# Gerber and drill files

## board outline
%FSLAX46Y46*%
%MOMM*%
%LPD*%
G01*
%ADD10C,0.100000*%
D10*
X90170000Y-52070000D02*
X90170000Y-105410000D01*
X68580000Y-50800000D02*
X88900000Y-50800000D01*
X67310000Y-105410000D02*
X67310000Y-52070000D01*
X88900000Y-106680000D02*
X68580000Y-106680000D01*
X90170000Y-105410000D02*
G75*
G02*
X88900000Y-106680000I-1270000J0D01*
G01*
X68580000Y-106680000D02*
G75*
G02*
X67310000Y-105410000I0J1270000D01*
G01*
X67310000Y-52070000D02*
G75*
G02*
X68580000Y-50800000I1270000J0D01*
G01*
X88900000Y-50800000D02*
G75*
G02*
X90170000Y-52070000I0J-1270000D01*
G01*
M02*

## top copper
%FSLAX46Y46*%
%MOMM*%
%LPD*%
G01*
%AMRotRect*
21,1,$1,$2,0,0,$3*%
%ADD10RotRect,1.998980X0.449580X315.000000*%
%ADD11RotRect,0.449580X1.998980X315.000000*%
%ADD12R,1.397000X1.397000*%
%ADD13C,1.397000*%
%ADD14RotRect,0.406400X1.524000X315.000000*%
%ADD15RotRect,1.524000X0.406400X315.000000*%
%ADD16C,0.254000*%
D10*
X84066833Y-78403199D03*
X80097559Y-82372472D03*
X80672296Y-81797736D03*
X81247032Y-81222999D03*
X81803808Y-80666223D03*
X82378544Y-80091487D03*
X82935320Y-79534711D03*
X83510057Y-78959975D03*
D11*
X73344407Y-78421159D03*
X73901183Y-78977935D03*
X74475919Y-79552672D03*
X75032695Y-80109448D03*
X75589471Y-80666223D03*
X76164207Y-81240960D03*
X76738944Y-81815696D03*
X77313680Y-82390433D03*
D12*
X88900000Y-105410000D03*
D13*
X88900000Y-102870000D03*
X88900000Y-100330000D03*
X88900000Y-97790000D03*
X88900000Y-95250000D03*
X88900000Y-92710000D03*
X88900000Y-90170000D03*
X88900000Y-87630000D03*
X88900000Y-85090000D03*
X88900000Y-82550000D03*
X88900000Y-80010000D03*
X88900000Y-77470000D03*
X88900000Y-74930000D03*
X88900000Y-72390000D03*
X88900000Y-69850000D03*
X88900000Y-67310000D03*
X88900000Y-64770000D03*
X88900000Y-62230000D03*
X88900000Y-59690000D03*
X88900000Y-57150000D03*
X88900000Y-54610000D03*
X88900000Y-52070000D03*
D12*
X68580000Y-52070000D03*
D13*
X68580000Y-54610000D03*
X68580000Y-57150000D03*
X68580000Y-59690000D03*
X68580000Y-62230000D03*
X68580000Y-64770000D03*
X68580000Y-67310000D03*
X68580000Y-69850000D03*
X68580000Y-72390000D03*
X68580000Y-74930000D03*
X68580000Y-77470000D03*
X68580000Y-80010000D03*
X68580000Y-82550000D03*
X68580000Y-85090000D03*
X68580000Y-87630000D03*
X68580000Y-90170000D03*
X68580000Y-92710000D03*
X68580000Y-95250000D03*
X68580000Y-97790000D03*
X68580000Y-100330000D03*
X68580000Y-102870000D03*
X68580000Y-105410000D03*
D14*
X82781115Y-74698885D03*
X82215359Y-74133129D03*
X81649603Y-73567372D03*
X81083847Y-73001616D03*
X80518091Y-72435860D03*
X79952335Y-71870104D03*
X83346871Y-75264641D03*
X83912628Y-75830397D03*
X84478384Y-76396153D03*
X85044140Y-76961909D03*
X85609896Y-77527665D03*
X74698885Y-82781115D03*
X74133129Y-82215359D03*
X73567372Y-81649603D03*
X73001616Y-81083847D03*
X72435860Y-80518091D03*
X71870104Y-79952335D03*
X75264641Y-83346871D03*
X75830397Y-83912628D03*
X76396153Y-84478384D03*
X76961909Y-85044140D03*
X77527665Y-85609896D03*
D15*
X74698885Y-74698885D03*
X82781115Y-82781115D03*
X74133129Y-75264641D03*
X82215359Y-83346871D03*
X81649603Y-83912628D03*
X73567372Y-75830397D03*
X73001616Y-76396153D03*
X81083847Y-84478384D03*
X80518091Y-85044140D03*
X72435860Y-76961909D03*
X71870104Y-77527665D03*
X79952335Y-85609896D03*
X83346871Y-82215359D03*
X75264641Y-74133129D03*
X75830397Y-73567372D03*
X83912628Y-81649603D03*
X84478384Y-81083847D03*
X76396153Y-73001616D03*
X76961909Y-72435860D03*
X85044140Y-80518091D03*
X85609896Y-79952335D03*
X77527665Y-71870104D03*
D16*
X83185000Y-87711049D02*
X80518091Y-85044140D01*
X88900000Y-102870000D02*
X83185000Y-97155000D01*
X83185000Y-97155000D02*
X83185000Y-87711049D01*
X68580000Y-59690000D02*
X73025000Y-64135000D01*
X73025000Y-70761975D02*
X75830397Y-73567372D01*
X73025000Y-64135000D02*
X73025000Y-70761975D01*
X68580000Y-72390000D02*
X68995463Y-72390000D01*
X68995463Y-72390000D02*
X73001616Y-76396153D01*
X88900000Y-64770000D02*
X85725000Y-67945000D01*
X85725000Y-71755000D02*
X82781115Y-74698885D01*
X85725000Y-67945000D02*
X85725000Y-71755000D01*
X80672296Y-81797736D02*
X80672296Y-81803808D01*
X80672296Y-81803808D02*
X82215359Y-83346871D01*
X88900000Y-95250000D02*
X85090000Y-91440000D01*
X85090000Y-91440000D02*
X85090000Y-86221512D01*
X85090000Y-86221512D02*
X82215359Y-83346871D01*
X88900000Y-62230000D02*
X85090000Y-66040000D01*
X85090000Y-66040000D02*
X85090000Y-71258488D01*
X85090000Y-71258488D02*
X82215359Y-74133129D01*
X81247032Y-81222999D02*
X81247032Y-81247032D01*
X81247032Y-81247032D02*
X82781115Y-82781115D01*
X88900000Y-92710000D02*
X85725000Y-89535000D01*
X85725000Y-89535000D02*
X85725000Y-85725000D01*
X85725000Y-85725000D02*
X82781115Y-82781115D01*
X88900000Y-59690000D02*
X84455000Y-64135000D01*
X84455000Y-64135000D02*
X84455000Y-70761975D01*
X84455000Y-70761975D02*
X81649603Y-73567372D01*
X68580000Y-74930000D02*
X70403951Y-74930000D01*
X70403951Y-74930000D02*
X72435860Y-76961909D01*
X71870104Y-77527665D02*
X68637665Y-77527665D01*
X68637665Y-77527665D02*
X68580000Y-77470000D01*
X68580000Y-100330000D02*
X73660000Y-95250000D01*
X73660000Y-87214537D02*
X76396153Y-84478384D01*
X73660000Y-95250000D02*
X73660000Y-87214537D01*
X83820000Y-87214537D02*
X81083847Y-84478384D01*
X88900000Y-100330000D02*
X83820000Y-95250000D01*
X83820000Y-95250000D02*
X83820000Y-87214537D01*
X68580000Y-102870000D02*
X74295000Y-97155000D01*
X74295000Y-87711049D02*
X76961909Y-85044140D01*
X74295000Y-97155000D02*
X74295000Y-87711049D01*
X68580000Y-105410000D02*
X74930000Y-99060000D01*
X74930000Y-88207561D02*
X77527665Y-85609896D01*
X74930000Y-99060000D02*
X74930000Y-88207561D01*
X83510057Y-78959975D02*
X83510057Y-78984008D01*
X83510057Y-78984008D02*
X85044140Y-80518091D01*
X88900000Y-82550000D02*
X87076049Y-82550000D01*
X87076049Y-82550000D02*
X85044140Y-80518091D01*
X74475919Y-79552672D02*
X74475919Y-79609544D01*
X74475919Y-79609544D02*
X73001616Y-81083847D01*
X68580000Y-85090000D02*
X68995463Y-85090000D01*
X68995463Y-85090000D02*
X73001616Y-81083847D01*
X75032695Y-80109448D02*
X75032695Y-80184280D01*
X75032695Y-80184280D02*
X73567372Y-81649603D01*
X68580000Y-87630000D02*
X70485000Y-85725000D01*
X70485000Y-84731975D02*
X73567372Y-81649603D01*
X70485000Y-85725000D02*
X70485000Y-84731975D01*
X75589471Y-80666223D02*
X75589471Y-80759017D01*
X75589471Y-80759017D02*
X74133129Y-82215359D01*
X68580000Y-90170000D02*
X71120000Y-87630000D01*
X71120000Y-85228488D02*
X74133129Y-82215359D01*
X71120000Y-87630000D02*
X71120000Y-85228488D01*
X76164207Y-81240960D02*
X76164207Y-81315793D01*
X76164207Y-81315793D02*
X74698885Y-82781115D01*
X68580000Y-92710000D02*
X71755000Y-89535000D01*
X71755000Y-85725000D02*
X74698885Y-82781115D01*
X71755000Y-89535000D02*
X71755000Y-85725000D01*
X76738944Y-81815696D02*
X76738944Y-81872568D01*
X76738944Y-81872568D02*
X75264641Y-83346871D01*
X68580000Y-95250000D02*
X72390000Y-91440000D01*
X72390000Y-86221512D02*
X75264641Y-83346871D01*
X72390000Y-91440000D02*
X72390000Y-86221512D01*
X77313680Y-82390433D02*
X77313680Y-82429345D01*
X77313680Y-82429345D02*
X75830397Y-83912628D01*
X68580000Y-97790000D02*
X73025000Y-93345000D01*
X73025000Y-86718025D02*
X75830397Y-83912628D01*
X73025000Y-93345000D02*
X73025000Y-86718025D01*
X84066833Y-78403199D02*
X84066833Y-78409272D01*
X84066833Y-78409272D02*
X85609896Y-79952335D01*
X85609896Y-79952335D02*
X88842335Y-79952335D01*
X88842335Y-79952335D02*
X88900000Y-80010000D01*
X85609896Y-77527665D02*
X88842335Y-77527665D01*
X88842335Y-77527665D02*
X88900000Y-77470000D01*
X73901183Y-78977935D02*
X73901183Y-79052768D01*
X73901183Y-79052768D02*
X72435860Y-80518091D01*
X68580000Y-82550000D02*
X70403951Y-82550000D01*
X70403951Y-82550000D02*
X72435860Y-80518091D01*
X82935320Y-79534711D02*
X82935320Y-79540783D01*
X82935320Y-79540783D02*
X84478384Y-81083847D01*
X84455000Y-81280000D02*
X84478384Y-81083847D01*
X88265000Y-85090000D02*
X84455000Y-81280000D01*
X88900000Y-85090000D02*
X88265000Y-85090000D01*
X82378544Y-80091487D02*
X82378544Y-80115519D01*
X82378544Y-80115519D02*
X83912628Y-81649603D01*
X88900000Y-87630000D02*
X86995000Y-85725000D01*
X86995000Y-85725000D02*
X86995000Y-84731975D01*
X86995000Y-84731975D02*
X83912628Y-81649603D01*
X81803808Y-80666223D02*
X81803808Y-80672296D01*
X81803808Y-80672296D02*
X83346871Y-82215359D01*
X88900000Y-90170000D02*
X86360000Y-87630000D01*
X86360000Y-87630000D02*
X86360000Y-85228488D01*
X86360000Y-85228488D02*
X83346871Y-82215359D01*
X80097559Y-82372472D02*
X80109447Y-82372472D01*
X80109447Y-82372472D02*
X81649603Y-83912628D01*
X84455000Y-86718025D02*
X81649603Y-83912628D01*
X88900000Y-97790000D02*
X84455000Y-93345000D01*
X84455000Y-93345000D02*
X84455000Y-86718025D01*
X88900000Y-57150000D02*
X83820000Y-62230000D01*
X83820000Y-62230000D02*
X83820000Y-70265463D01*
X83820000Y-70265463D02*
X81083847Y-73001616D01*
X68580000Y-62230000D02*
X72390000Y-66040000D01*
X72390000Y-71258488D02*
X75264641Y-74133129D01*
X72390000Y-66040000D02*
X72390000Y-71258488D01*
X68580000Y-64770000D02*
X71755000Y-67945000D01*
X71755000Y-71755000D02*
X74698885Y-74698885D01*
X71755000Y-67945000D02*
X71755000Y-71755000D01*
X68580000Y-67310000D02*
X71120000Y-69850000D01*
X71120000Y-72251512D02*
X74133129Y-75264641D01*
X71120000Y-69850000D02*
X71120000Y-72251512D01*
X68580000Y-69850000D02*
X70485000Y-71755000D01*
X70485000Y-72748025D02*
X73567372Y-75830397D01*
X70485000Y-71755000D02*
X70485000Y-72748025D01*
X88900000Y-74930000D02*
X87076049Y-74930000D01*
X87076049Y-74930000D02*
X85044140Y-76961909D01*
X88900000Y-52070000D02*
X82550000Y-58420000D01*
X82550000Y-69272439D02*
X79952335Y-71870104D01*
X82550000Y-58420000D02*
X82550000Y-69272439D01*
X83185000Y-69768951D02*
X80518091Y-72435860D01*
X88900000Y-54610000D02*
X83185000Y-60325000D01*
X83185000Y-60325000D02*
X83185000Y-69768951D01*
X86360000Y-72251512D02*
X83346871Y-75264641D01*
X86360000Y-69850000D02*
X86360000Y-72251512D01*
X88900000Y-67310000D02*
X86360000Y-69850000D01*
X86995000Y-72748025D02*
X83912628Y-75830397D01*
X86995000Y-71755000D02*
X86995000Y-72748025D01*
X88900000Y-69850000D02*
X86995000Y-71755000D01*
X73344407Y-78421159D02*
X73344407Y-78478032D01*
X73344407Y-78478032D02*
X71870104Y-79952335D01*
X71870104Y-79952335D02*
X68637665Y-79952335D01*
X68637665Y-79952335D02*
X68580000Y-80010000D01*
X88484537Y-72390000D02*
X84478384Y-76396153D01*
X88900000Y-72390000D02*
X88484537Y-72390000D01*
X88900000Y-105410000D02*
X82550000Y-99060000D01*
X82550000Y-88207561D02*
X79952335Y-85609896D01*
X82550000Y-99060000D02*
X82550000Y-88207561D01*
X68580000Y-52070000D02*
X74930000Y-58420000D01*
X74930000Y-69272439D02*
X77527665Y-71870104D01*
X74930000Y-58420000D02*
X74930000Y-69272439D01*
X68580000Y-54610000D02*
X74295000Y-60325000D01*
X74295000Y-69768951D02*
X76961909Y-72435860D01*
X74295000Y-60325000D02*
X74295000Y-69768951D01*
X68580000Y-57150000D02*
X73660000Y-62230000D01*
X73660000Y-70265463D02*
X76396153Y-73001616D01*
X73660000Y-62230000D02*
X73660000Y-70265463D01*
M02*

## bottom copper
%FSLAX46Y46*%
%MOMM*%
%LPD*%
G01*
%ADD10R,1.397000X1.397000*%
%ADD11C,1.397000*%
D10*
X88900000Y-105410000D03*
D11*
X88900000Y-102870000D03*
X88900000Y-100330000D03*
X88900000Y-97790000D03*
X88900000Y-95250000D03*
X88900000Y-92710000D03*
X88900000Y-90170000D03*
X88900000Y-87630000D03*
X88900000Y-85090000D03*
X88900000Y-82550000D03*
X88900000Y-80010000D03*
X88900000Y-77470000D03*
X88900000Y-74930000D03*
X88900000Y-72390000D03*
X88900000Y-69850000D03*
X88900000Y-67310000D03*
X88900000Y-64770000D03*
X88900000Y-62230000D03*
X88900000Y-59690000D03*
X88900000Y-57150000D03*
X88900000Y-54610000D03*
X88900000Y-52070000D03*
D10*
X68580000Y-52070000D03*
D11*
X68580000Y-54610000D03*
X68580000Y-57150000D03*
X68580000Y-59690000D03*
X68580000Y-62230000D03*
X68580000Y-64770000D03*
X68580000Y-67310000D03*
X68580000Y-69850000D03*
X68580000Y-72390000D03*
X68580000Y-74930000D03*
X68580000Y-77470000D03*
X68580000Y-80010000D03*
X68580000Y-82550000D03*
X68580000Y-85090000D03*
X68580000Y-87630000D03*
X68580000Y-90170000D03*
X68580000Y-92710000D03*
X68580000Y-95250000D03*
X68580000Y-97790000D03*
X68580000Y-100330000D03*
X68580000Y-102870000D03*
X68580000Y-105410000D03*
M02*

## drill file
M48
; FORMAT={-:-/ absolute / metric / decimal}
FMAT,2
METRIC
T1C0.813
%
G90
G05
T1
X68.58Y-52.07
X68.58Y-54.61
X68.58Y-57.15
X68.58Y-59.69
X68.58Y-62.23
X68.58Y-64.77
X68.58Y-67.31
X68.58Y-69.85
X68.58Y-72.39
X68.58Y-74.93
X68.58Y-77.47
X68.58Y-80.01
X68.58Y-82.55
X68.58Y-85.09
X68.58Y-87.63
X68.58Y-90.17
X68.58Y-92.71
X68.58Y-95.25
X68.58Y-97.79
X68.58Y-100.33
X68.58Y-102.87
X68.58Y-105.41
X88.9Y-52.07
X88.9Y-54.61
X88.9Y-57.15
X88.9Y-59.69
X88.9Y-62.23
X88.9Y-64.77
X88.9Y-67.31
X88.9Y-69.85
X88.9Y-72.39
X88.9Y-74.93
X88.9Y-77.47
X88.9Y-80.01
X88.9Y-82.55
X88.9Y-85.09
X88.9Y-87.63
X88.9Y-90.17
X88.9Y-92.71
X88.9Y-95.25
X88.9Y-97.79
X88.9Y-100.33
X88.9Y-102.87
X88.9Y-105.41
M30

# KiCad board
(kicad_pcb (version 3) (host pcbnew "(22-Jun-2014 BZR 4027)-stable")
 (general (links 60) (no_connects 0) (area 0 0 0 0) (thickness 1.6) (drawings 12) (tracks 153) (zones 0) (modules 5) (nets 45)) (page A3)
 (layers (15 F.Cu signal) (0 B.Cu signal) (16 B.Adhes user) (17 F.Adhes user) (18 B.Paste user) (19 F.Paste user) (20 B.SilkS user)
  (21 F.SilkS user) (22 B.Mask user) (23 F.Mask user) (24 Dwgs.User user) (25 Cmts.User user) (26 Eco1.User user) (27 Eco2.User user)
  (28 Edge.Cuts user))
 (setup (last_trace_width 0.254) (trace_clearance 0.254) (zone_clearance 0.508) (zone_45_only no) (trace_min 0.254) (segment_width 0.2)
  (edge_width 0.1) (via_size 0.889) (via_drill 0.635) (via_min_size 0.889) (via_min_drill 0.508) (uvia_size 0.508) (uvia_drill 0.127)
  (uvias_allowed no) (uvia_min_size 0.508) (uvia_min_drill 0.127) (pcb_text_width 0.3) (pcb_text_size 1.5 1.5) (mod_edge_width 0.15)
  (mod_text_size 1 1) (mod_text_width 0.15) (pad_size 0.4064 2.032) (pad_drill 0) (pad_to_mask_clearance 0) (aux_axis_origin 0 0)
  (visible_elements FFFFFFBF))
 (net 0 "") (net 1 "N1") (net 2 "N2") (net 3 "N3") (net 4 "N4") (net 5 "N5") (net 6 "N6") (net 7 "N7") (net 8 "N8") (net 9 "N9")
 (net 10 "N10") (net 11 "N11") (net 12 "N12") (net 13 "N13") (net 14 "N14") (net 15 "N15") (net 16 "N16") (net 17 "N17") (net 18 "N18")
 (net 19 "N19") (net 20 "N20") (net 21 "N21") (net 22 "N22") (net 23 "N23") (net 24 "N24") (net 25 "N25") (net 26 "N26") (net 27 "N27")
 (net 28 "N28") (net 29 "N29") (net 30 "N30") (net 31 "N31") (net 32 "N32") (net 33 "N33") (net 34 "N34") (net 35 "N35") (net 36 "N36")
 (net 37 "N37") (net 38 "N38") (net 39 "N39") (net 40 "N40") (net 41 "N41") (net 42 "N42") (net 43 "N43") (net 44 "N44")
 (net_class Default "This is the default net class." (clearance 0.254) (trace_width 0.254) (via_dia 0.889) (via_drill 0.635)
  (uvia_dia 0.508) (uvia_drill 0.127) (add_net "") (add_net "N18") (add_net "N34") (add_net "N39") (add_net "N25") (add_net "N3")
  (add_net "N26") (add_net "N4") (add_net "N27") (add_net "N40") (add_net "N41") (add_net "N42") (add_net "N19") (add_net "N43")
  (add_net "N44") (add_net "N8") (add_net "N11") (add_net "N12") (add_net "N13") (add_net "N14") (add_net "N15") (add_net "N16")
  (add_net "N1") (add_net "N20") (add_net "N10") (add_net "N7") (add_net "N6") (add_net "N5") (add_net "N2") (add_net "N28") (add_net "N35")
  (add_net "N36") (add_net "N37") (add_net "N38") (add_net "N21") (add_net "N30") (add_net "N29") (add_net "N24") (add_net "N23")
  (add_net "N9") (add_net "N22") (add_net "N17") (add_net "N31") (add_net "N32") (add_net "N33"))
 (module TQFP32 (layer F.Cu) (at 78.7146 77.0382 315)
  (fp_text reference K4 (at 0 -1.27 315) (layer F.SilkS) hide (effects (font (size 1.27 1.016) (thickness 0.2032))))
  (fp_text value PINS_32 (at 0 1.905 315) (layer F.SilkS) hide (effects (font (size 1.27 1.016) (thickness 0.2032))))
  (pad 24 smd rect (at 4.7498 -2.8194 315) (size 1.99898 0.44958) (layers F.Cu F.Paste F.Mask) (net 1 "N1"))
  (pad 17 smd rect (at 4.7498 2.794 315) (size 1.99898 0.44958) (layers F.Cu F.Paste F.Mask) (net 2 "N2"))
  (pad 18 smd rect (at 4.7498 1.9812 315) (size 1.99898 0.44958) (layers F.Cu F.Paste F.Mask) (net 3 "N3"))
  (pad 19 smd rect (at 4.7498 1.1684 315) (size 1.99898 0.44958) (layers F.Cu F.Paste F.Mask) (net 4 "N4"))
  (pad 20 smd rect (at 4.7498 0.381 315) (size 1.99898 0.44958) (layers F.Cu F.Paste F.Mask) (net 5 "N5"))
  (pad 21 smd rect (at 4.7498 -0.4318 315) (size 1.99898 0.44958) (layers F.Cu F.Paste F.Mask) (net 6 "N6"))
  (pad 22 smd rect (at 4.7498 -1.2192 315) (size 1.99898 0.44958) (layers F.Cu F.Paste F.Mask) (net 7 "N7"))
  (pad 23 smd rect (at 4.7498 -2.032 315) (size 1.99898 0.44958) (layers F.Cu F.Paste F.Mask) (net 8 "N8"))
  (pad 9 smd rect (at -2.8194 4.7752 315) (size 0.44958 1.99898) (layers F.Cu F.Paste F.Mask) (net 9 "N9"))
  (pad 10 smd rect (at -2.032 4.7752 315) (size 0.44958 1.99898) (layers F.Cu F.Paste F.Mask) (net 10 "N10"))
  (pad 11 smd rect (at -1.2192 4.7752 315) (size 0.44958 1.99898) (layers F.Cu F.Paste F.Mask) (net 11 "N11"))
  (pad 12 smd rect (at -0.4318 4.7752 315) (size 0.44958 1.99898) (layers F.Cu F.Paste F.Mask) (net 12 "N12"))
  (pad 13 smd rect (at 0.3556 4.7752 315) (size 0.44958 1.99898) (layers F.Cu F.Paste F.Mask) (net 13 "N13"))
  (pad 14 smd rect (at 1.1684 4.7752 315) (size 0.44958 1.99898) (layers F.Cu F.Paste F.Mask) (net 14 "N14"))
  (pad 15 smd rect (at 1.9812 4.7752 315) (size 0.44958 1.99898) (layers F.Cu F.Paste F.Mask) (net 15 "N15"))
  (pad 16 smd rect (at 2.794 4.7752 315) (size 0.44958 1.99898) (layers F.Cu F.Paste F.Mask) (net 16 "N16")))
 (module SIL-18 (layer F.Cu) (at 88.9 83.82 90)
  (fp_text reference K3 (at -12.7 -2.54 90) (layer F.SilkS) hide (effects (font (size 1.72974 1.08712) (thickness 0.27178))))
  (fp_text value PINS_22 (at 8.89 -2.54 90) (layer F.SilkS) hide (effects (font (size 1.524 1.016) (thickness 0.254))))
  (pad 1 thru_hole rect (at -21.59 0 90) (size 1.397 1.397) (drill 0.8128) (layers *.Cu *.Mask F.SilkS) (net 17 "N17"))
  (pad 2 thru_hole circle (at -19.05 0 90) (size 1.397 1.397) (drill 0.8128) (layers *.Cu *.Mask F.SilkS) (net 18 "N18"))
  (pad 3 thru_hole circle (at -16.51 0 90) (size 1.397 1.397) (drill 0.8128) (layers *.Cu *.Mask F.SilkS) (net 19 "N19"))
  (pad 4 thru_hole circle (at -13.97 0 90) (size 1.397 1.397) (drill 0.8128) (layers *.Cu *.Mask F.SilkS) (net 2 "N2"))
  (pad 5 thru_hole circle (at -11.43 0 90) (size 1.397 1.397) (drill 0.8128) (layers *.Cu *.Mask F.SilkS) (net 3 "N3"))
  (pad 6 thru_hole circle (at -8.89 0 90) (size 1.397 1.397) (drill 0.8128) (layers *.Cu *.Mask F.SilkS) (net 4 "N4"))
  (pad 7 thru_hole circle (at -6.35 0 90) (size 1.397 1.397) (drill 0.8128) (layers *.Cu *.Mask F.SilkS) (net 5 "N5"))
  (pad 8 thru_hole circle (at -3.81 0 90) (size 1.397 1.397) (drill 0.8128) (layers *.Cu *.Mask F.SilkS) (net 6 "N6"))
  (pad 9 thru_hole circle (at -1.27 0 90) (size 1.397 1.397) (drill 0.8128) (layers *.Cu *.Mask F.SilkS) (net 7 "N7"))
  (pad 10 thru_hole circle (at 1.27 0 90) (size 1.397 1.397) (drill 0.8128) (layers *.Cu *.Mask F.SilkS) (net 8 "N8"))
  (pad 11 thru_hole circle (at 3.81 0 90) (size 1.397 1.397) (drill 0.8128) (layers *.Cu *.Mask F.SilkS) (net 1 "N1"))
  (pad 12 thru_hole circle (at 6.35 0 90) (size 1.397 1.397) (drill 0.8128) (layers *.Cu *.Mask F.SilkS) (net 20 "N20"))
  (pad 13 thru_hole circle (at 8.89 0 90) (size 1.397 1.397) (drill 0.8128) (layers *.Cu *.Mask F.SilkS) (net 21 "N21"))
  (pad 14 thru_hole circle (at 11.43 0 90) (size 1.397 1.397) (drill 0.8128) (layers *.Cu *.Mask F.SilkS) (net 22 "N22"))
  (pad 15 thru_hole circle (at 13.97 0 90) (size 1.397 1.397) (drill 0.8128) (layers *.Cu *.Mask F.SilkS) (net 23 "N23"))
  (pad 16 thru_hole circle (at 16.51 0 90) (size 1.397 1.397) (drill 0.8128) (layers *.Cu *.Mask F.SilkS) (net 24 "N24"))
  (pad 17 thru_hole circle (at 19.05 0 90) (size 1.397 1.397) (drill 0.8128) (layers *.Cu *.Mask F.SilkS) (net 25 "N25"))
  (pad 18 thru_hole circle (at 21.59 0 90) (size 1.397 1.397) (drill 0.8128) (layers *.Cu *.Mask F.SilkS) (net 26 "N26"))
  (pad 19 thru_hole circle (at 24.13 0 90) (size 1.397 1.397) (drill 0.8128) (layers *.Cu *.Mask F.SilkS) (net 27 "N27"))
  (pad 20 thru_hole circle (at 26.67 0 90) (size 1.397 1.397) (drill 0.8128) (layers *.Cu *.Mask F.SilkS) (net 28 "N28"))
  (pad 21 thru_hole circle (at 29.21 0 90) (size 1.397 1.397) (drill 0.8128) (layers *.Cu *.Mask F.SilkS) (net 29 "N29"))
  (pad 22 thru_hole circle (at 31.75 0 90) (size 1.397 1.397) (drill 0.8128) (layers *.Cu *.Mask F.SilkS) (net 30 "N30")))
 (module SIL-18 (layer F.Cu) (at 68.58 73.66 270)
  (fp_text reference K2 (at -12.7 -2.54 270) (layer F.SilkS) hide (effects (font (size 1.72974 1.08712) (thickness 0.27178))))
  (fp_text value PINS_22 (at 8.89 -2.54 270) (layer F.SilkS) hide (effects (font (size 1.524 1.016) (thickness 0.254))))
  (pad 1 thru_hole rect (at -21.59 0 270) (size 1.397 1.397) (drill 0.8128) (layers *.Cu *.Mask F.SilkS) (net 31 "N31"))
  (pad 2 thru_hole circle (at -19.05 0 270) (size 1.397 1.397) (drill 0.8128) (layers *.Cu *.Mask F.SilkS) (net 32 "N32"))
  (pad 3 thru_hole circle (at -16.51 0 270) (size 1.397 1.397) (drill 0.8128) (layers *.Cu *.Mask F.SilkS) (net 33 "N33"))
  (pad 4 thru_hole circle (at -13.97 0 270) (size 1.397 1.397) (drill 0.8128) (layers *.Cu *.Mask F.SilkS) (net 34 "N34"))
  (pad 5 thru_hole circle (at -11.43 0 270) (size 1.397 1.397) (drill 0.8128) (layers *.Cu *.Mask F.SilkS) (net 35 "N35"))
  (pad 6 thru_hole circle (at -8.89 0 270) (size 1.397 1.397) (drill 0.8128) (layers *.Cu *.Mask F.SilkS) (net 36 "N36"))
  (pad 7 thru_hole circle (at -6.35 0 270) (size 1.397 1.397) (drill 0.8128) (layers *.Cu *.Mask F.SilkS) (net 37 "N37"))
  (pad 8 thru_hole circle (at -3.81 0 270) (size 1.397 1.397) (drill 0.8128) (layers *.Cu *.Mask F.SilkS) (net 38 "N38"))
  (pad 9 thru_hole circle (at -1.27 0 270) (size 1.397 1.397) (drill 0.8128) (layers *.Cu *.Mask F.SilkS) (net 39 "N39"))
  (pad 10 thru_hole circle (at 1.27 0 270) (size 1.397 1.397) (drill 0.8128) (layers *.Cu *.Mask F.SilkS) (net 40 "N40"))
  (pad 11 thru_hole circle (at 3.81 0 270) (size 1.397 1.397) (drill 0.8128) (layers *.Cu *.Mask F.SilkS) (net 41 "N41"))
  (pad 12 thru_hole circle (at 6.35 0 270) (size 1.397 1.397) (drill 0.8128) (layers *.Cu *.Mask F.SilkS) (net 9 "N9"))
  (pad 13 thru_hole circle (at 8.89 0 270) (size 1.397 1.397) (drill 0.8128) (layers *.Cu *.Mask F.SilkS) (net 10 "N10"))
  (pad 14 thru_hole circle (at 11.43 0 270) (size 1.397 1.397) (drill 0.8128) (layers *.Cu *.Mask F.SilkS) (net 11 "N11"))
  (pad 15 thru_hole circle (at 13.97 0 270) (size 1.397 1.397) (drill 0.8128) (layers *.Cu *.Mask F.SilkS) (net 12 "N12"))
  (pad 16 thru_hole circle (at 16.51 0 270) (size 1.397 1.397) (drill 0.8128) (layers *.Cu *.Mask F.SilkS) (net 13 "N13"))
  (pad 17 thru_hole circle (at 19.05 0 270) (size 1.397 1.397) (drill 0.8128) (layers *.Cu *.Mask F.SilkS) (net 14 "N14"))
  (pad 18 thru_hole circle (at 21.59 0 270) (size 1.397 1.397) (drill 0.8128) (layers *.Cu *.Mask F.SilkS) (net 15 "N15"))
  (pad 19 thru_hole circle (at 24.13 0 270) (size 1.397 1.397) (drill 0.8128) (layers *.Cu *.Mask F.SilkS) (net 16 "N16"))
  (pad 20 thru_hole circle (at 26.67 0 270) (size 1.397 1.397) (drill 0.8128) (layers *.Cu *.Mask F.SilkS) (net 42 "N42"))
  (pad 21 thru_hole circle (at 29.21 0 270) (size 1.397 1.397) (drill 0.8128) (layers *.Cu *.Mask F.SilkS) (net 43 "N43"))
  (pad 22 thru_hole circle (at 31.75 0 270) (size 1.397 1.397) (drill 0.8128) (layers *.Cu *.Mask F.SilkS) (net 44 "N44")))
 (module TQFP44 (layer F.Cu) (at 78.74 78.74 315)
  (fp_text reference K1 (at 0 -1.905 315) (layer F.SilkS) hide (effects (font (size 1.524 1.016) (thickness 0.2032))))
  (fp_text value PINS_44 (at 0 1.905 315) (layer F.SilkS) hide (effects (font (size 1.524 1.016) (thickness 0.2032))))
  (pad 39 smd rect (at 0 -5.715 315) (size 0.4064 1.524) (layers F.Cu F.Paste F.Mask) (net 25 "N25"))
  (pad 40 smd rect (at -0.8001 -5.715 315) (size 0.4064 1.524) (layers F.Cu F.Paste F.Mask) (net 26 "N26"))
  (pad 41 smd rect (at -1.6002 -5.715 315) (size 0.4064 1.524) (layers F.Cu F.Paste F.Mask) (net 27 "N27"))
  (pad 42 smd rect (at -2.4003 -5.715 315) (size 0.4064 1.524) (layers F.Cu F.Paste F.Mask) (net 28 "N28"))
  (pad 43 smd rect (at -3.2004 -5.715 315) (size 0.4064 1.524) (layers F.Cu F.Paste F.Mask) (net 29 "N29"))
  (pad 44 smd rect (at -4.0005 -5.715 315) (size 0.4064 1.524) (layers F.Cu F.Paste F.Mask) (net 30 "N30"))
  (pad 38 smd rect (at 0.8001 -5.715 315) (size 0.4064 1.524) (layers F.Cu F.Paste F.Mask) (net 24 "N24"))
  (pad 37 smd rect (at 1.6002 -5.715 315) (size 0.4064 1.524) (layers F.Cu F.Paste F.Mask) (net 23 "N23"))
  (pad 36 smd rect (at 2.4003 -5.715 315) (size 0.4064 1.524) (layers F.Cu F.Paste F.Mask) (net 22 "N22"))
  (pad 35 smd rect (at 3.2004 -5.715 315) (size 0.4064 1.524) (layers F.Cu F.Paste F.Mask) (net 21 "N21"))
  (pad 34 smd rect (at 4.0005 -5.715 315) (size 0.4064 1.524) (layers F.Cu F.Paste F.Mask) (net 20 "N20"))
  (pad 17 smd rect (at 0 5.715 315) (size 0.4064 1.524) (layers F.Cu F.Paste F.Mask) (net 14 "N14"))
  (pad 16 smd rect (at -0.8001 5.715 315) (size 0.4064 1.524) (layers F.Cu F.Paste F.Mask) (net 13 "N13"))
  (pad 15 smd rect (at -1.6002 5.715 315) (size 0.4064 1.524) (layers F.Cu F.Paste F.Mask) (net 12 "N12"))
  (pad 14 smd rect (at -2.4003 5.715 315) (size 0.4064 1.524) (layers F.Cu F.Paste F.Mask) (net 11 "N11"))
  (pad 13 smd rect (at -3.2004 5.715 315) (size 0.4064 1.524) (layers F.Cu F.Paste F.Mask) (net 10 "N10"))
  (pad 12 smd rect (at -4.0005 5.715 315) (size 0.4064 1.524) (layers F.Cu F.Paste F.Mask) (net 9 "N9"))
  (pad 18 smd rect (at 0.8001 5.715 315) (size 0.4064 1.524) (layers F.Cu F.Paste F.Mask) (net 15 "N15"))
  (pad 19 smd rect (at 1.6002 5.715 315) (size 0.4064 1.524) (layers F.Cu F.Paste F.Mask) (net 16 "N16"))
  (pad 20 smd rect (at 2.4003 5.715 315) (size 0.4064 1.524) (layers F.Cu F.Paste F.Mask) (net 42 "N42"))
  (pad 21 smd rect (at 3.2004 5.715 315) (size 0.4064 1.524) (layers F.Cu F.Paste F.Mask) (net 43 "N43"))
  (pad 22 smd rect (at 4.0005 5.715 315) (size 0.4064 1.524) (layers F.Cu F.Paste F.Mask) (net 44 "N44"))
  (pad 6 smd rect (at -5.715 0 315) (size 1.524 0.4064) (layers F.Cu F.Paste F.Mask) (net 36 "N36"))
  (pad 28 smd rect (at 5.715 0 315) (size 1.524 0.4064) (layers F.Cu F.Paste F.Mask) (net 4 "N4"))
  (pad 7 smd rect (at -5.715 0.8001 315) (size 1.524 0.4064) (layers F.Cu F.Paste F.Mask) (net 37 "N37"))
  (pad 27 smd rect (at 5.715 0.8001 315) (size 1.524 0.4064) (layers F.Cu F.Paste F.Mask) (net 3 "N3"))
  (pad 26 smd rect (at 5.715 1.6002 315) (size 1.524 0.4064) (layers F.Cu F.Paste F.Mask) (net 2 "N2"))
  (pad 8 smd rect (at -5.715 1.6002 315) (size 1.524 0.4064) (layers F.Cu F.Paste F.Mask) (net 38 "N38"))
  (pad 9 smd rect (at -5.715 2.4003 315) (size 1.524 0.4064) (layers F.Cu F.Paste F.Mask) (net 39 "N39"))
  (pad 25 smd rect (at 5.715 2.4003 315) (size 1.524 0.4064) (layers F.Cu F.Paste F.Mask) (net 19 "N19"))
  (pad 24 smd rect (at 5.715 3.2004 315) (size 1.524 0.4064) (layers F.Cu F.Paste F.Mask) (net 18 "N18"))
  (pad 10 smd rect (at -5.715 3.2004 315) (size 1.524 0.4064) (layers F.Cu F.Paste F.Mask) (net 40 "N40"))
  (pad 11 smd rect (at -5.715 4.0005 315) (size 1.524 0.4064) (layers F.Cu F.Paste F.Mask) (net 41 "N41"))
  (pad 23 smd rect (at 5.715 4.0005 315) (size 1.524 0.4064) (layers F.Cu F.Paste F.Mask) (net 17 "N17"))
  (pad 29 smd rect (at 5.715 -0.8001 315) (size 1.524 0.4064) (layers F.Cu F.Paste F.Mask) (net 5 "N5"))
  (pad 5 smd rect (at -5.715 -0.8001 315) (size 1.524 0.4064) (layers F.Cu F.Paste F.Mask) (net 35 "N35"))
  (pad 4 smd rect (at -5.715 -1.6002 315) (size 1.524 0.4064) (layers F.Cu F.Paste F.Mask) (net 34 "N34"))
  (pad 30 smd rect (at 5.715 -1.6002 315) (size 1.524 0.4064) (layers F.Cu F.Paste F.Mask) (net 6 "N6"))
  (pad 31 smd rect (at 5.715 -2.4003 315) (size 1.524 0.4064) (layers F.Cu F.Paste F.Mask) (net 7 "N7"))
  (pad 3 smd rect (at -5.715 -2.4003 315) (size 1.524 0.4064) (layers F.Cu F.Paste F.Mask) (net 33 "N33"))
  (pad 2 smd rect (at -5.715 -3.2004 315) (size 1.524 0.4064) (layers F.Cu F.Paste F.Mask) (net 32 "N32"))
  (pad 32 smd rect (at 5.715 -3.2004 315) (size 1.524 0.4064) (layers F.Cu F.Paste F.Mask) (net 8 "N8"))
  (pad 33 smd rect (at 5.715 -4.0005 315) (size 1.524 0.4064) (layers F.Cu F.Paste F.Mask) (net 1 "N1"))
  (pad 1 smd rect (at -5.715 -4.0005 315) (size 1.524 0.4064) (layers F.Cu F.Paste F.Mask) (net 31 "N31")))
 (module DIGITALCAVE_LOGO (layer F.Cu) (at 78.74 93.98 90)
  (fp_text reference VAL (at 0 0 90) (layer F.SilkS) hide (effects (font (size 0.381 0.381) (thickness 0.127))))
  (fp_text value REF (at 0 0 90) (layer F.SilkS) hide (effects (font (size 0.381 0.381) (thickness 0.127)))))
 (gr_line (start 90.17 52.07) (end 90.17 105.41) (angle 90) (layer Edge.Cuts) (width 0.1))
 (gr_line (start 68.58 50.8) (end 88.9 50.8) (angle 90) (layer Edge.Cuts) (width 0.1))
 (gr_line (start 67.31 105.41) (end 67.31 52.07) (angle 90) (layer Edge.Cuts) (width 0.1))
 (gr_line (start 88.9 106.68) (end 68.58 106.68) (angle 90) (layer Edge.Cuts) (width 0.1))
 (gr_arc (start 88.9 105.41) (end 90.17 105.41) (angle 90) (layer Edge.Cuts) (width 0.1))
 (gr_arc (start 68.58 105.41) (end 68.58 106.68) (angle 90) (layer Edge.Cuts) (width 0.1))
 (gr_arc (start 68.58 52.07) (end 67.31 52.07) (angle 90) (layer Edge.Cuts) (width 0.1))
 (gr_arc (start 88.9 52.07) (end 88.9 50.8) (angle 90) (layer Edge.Cuts) (width 0.1))
 (segment (start 83.185 87.711049) (end 80.518091 85.04414) (width 0.254) (layer F.Cu) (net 18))
 (segment (start 88.9 102.87) (end 83.185 97.155) (width 0.254) (layer F.Cu) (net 18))
 (segment (start 83.185 97.155) (end 83.185 87.711049) (width 0.254) (layer F.Cu) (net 18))
 (segment (start 68.58 59.69) (end 73.025 64.135) (width 0.254) (layer F.Cu) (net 34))
 (segment (start 73.025 70.761975) (end 75.830397 73.567372) (width 0.254) (layer F.Cu) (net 34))
 (segment (start 73.025 64.135) (end 73.025 70.761975) (width 0.254) (layer F.Cu) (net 34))
 (segment (start 68.58 72.39) (end 68.995463 72.39) (width 0.254) (layer F.Cu) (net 39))
 (segment (start 68.995463 72.39) (end 73.001616 76.396153) (width 0.254) (layer F.Cu) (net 39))
 (segment (start 88.9 64.77) (end 85.725 67.945) (width 0.254) (layer F.Cu) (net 25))
 (segment (start 85.725 71.755) (end 82.781115 74.698885) (width 0.254) (layer F.Cu) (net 25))
 (segment (start 85.725 67.945) (end 85.725 71.755) (width 0.254) (layer F.Cu) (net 25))
 (segment (start 80.672296 81.797736) (end 80.672296 81.803808) (width 0.254) (layer F.Cu) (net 3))
 (segment (start 80.672296 81.803808) (end 82.215359 83.346871) (width 0.254) (layer F.Cu) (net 3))
 (segment (start 88.9 95.25) (end 85.09 91.44) (width 0.254) (layer F.Cu) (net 3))
 (segment (start 85.09 91.44) (end 85.09 86.221512) (width 0.254) (layer F.Cu) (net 3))
 (segment (start 85.09 86.221512) (end 82.215359 83.346871) (width 0.254) (layer F.Cu) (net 3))
 (segment (start 88.9 62.23) (end 85.09 66.04) (width 0.254) (layer F.Cu) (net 26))
 (segment (start 85.09 66.04) (end 85.09 71.258488) (width 0.254) (layer F.Cu) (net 26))
 (segment (start 85.09 71.258488) (end 82.215359 74.133129) (width 0.254) (layer F.Cu) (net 26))
 (segment (start 81.247032 81.222999) (end 81.247032 81.247032) (width 0.254) (layer F.Cu) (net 4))
 (segment (start 81.247032 81.247032) (end 82.781115 82.781115) (width 0.254) (layer F.Cu) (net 4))
 (segment (start 88.9 92.71) (end 85.725 89.535) (width 0.254) (layer F.Cu) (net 4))
 (segment (start 85.725 89.535) (end 85.725 85.725) (width 0.254) (layer F.Cu) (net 4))
 (segment (start 85.725 85.725) (end 82.781115 82.781115) (width 0.254) (layer F.Cu) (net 4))
 (segment (start 88.9 59.69) (end 84.455 64.135) (width 0.254) (layer F.Cu) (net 27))
 (segment (start 84.455 64.135) (end 84.455 70.761975) (width 0.254) (layer F.Cu) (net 27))
 (segment (start 84.455 70.761975) (end 81.649603 73.567372) (width 0.254) (layer F.Cu) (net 27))
 (segment (start 68.58 74.93) (end 70.403951 74.93) (width 0.254) (layer F.Cu) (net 40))
 (segment (start 70.403951 74.93) (end 72.43586 76.961909) (width 0.254) (layer F.Cu) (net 40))
 (segment (start 71.870104 77.527665) (end 68.637665 77.527665) (width 0.254) (layer F.Cu) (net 41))
 (segment (start 68.637665 77.527665) (end 68.58 77.47) (width 0.254) (layer F.Cu) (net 41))
 (segment (start 68.58 100.33) (end 73.66 95.25) (width 0.254) (layer F.Cu) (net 42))
 (segment (start 73.66 87.214537) (end 76.396153 84.478384) (width 0.254) (layer F.Cu) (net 42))
 (segment (start 73.66 95.25) (end 73.66 87.214537) (width 0.254) (layer F.Cu) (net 42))
 (segment (start 83.82 87.214537) (end 81.083847 84.478384) (width 0.254) (layer F.Cu) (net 19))
 (segment (start 88.9 100.33) (end 83.82 95.25) (width 0.254) (layer F.Cu) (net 19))
 (segment (start 83.82 95.25) (end 83.82 87.214537) (width 0.254) (layer F.Cu) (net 19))
 (segment (start 68.58 102.87) (end 74.295 97.155) (width 0.254) (layer F.Cu) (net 43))
 (segment (start 74.295 87.711049) (end 76.961909 85.04414) (width 0.254) (layer F.Cu) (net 43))
 (segment (start 74.295 97.155) (end 74.295 87.711049) (width 0.254) (layer F.Cu) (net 43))
 (segment (start 68.58 105.41) (end 74.93 99.06) (width 0.254) (layer F.Cu) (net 44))
 (segment (start 74.93 88.207561) (end 77.527665 85.609896) (width 0.254) (layer F.Cu) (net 44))
 (segment (start 74.93 99.06) (end 74.93 88.207561) (width 0.254) (layer F.Cu) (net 44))
 (segment (start 83.510057 78.959975) (end 83.510057 78.984008) (width 0.254) (layer F.Cu) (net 8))
 (segment (start 83.510057 78.984008) (end 85.04414 80.518091) (width 0.254) (layer F.Cu) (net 8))
 (segment (start 88.9 82.55) (end 87.076049 82.55) (width 0.254) (layer F.Cu) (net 8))
 (segment (start 87.076049 82.55) (end 85.04414 80.518091) (width 0.254) (layer F.Cu) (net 8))
 (segment (start 74.475919 79.552672) (end 74.475919 79.609544) (width 0.254) (layer F.Cu) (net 11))
 (segment (start 74.475919 79.609544) (end 73.001616 81.083847) (width 0.254) (layer F.Cu) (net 11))
 (segment (start 68.58 85.09) (end 68.995463 85.09) (width 0.254) (layer F.Cu) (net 11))
 (segment (start 68.995463 85.09) (end 73.001616 81.083847) (width 0.254) (layer F.Cu) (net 11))
 (segment (start 75.032695 80.109448) (end 75.032695 80.18428) (width 0.254) (layer F.Cu) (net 12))
 (segment (start 75.032695 80.18428) (end 73.567372 81.649603) (width 0.254) (layer F.Cu) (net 12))
 (segment (start 68.58 87.63) (end 70.485 85.725) (width 0.254) (layer F.Cu) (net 12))
 (segment (start 70.485 84.731975) (end 73.567372 81.649603) (width 0.254) (layer F.Cu) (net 12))
 (segment (start 70.485 85.725) (end 70.485 84.731975) (width 0.254) (layer F.Cu) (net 12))
 (segment (start 75.589471 80.666223) (end 75.589471 80.759017) (width 0.254) (layer F.Cu) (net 13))
 (segment (start 75.589471 80.759017) (end 74.133129 82.215359) (width 0.254) (layer F.Cu) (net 13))
 (segment (start 68.58 90.17) (end 71.12 87.63) (width 0.254) (layer F.Cu) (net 13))
 (segment (start 71.12 85.228488) (end 74.133129 82.215359) (width 0.254) (layer F.Cu) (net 13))
 (segment (start 71.12 87.63) (end 71.12 85.228488) (width 0.254) (layer F.Cu) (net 13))
 (segment (start 76.164207 81.24096) (end 76.164207 81.315793) (width 0.254) (layer F.Cu) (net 14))
 (segment (start 76.164207 81.315793) (end 74.698885 82.781115) (width 0.254) (layer F.Cu) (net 14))
 (segment (start 68.58 92.71) (end 71.755 89.535) (width 0.254) (layer F.Cu) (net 14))
 (segment (start 71.755 85.725) (end 74.698885 82.781115) (width 0.254) (layer F.Cu) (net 14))
 (segment (start 71.755 89.535) (end 71.755 85.725) (width 0.254) (layer F.Cu) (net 14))
 (segment (start 76.738944 81.815696) (end 76.738944 81.872568) (width 0.254) (layer F.Cu) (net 15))
 (segment (start 76.738944 81.872568) (end 75.264641 83.346871) (width 0.254) (layer F.Cu) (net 15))
 (segment (start 68.58 95.25) (end 72.39 91.44) (width 0.254) (layer F.Cu) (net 15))
 (segment (start 72.39 86.221512) (end 75.264641 83.346871) (width 0.254) (layer F.Cu) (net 15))
 (segment (start 72.39 91.44) (end 72.39 86.221512) (width 0.254) (layer F.Cu) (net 15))
 (segment (start 77.31368 82.390433) (end 77.31368 82.429345) (width 0.254) (layer F.Cu) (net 16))
 (segment (start 77.31368 82.429345) (end 75.830397 83.912628) (width 0.254) (layer F.Cu) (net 16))
 (segment (start 68.58 97.79) (end 73.025 93.345) (width 0.254) (layer F.Cu) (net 16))
 (segment (start 73.025 86.718025) (end 75.830397 83.912628) (width 0.254) (layer F.Cu) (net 16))
 (segment (start 73.025 93.345) (end 73.025 86.718025) (width 0.254) (layer F.Cu) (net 16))
 (segment (start 84.066833 78.403199) (end 84.066833 78.409272) (width 0.254) (layer F.Cu) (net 1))
 (segment (start 84.066833 78.409272) (end 85.609896 79.952335) (width 0.254) (layer F.Cu) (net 1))
 (segment (start 85.609896 79.952335) (end 88.842335 79.952335) (width 0.254) (layer F.Cu) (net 1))
 (segment (start 88.842335 79.952335) (end 88.9 80.01) (width 0.254) (layer F.Cu) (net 1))
 (segment (start 85.609896 77.527665) (end 88.842335 77.527665) (width 0.254) (layer F.Cu) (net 20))
 (segment (start 88.842335 77.527665) (end 88.9 77.47) (width 0.254) (layer F.Cu) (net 20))
 (segment (start 73.901183 78.977935) (end 73.901183 79.052768) (width 0.254) (layer F.Cu) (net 10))
 (segment (start 73.901183 79.052768) (end 72.43586 80.518091) (width 0.254) (layer F.Cu) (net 10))
 (segment (start 68.58 82.55) (end 70.403951 82.55) (width 0.254) (layer F.Cu) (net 10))
 (segment (start 70.403951 82.55) (end 72.43586 80.518091) (width 0.254) (layer F.Cu) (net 10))
 (segment (start 82.93532 79.534711) (end 82.93532 79.540783) (width 0.254) (layer F.Cu) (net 7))
 (segment (start 82.93532 79.540783) (end 84.478384 81.083847) (width 0.254) (layer F.Cu) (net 7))
 (segment (start 84.455 81.28) (end 84.478384 81.083847) (width 0.254) (layer F.Cu) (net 7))
 (segment (start 88.265 85.09) (end 84.455 81.28) (width 0.254) (layer F.Cu) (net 7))
 (segment (start 88.9 85.09) (end 88.265 85.09) (width 0.254) (layer F.Cu) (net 7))
 (segment (start 82.378544 80.091487) (end 82.378544 80.115519) (width 0.254) (layer F.Cu) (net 6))
 (segment (start 82.378544 80.115519) (end 83.912628 81.649603) (width 0.254) (layer F.Cu) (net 6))
 (segment (start 88.9 87.63) (end 86.995 85.725) (width 0.254) (layer F.Cu) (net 6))
 (segment (start 86.995 85.725) (end 86.995 84.731975) (width 0.254) (layer F.Cu) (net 6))
 (segment (start 86.995 84.731975) (end 83.912628 81.649603) (width 0.254) (layer F.Cu) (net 6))
 (segment (start 81.803808 80.666223) (end 81.803808 80.672296) (width 0.254) (layer F.Cu) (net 5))
 (segment (start 81.803808 80.672296) (end 83.346871 82.215359) (width 0.254) (layer F.Cu) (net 5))
 (segment (start 88.9 90.17) (end 86.36 87.63) (width 0.254) (layer F.Cu) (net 5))
 (segment (start 86.36 87.63) (end 86.36 85.228488) (width 0.254) (layer F.Cu) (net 5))
 (segment (start 86.36 85.228488) (end 83.346871 82.215359) (width 0.254) (layer F.Cu) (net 5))
 (segment (start 80.097559 82.372472) (end 80.109447 82.372472) (width 0.254) (layer F.Cu) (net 2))
 (segment (start 80.109447 82.372472) (end 81.649603 83.912628) (width 0.254) (layer F.Cu) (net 2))
 (segment (start 84.455 86.718025) (end 81.649603 83.912628) (width 0.254) (layer F.Cu) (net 2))
 (segment (start 88.9 97.79) (end 84.455 93.345) (width 0.254) (layer F.Cu) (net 2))
 (segment (start 84.455 93.345) (end 84.455 86.718025) (width 0.254) (layer F.Cu) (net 2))
 (segment (start 88.9 57.15) (end 83.82 62.23) (width 0.254) (layer F.Cu) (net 28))
 (segment (start 83.82 62.23) (end 83.82 70.265463) (width 0.254) (layer F.Cu) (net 28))
 (segment (start 83.82 70.265463) (end 81.083847 73.001616) (width 0.254) (layer F.Cu) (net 28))
 (segment (start 68.58 62.23) (end 72.39 66.04) (width 0.254) (layer F.Cu) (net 35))
 (segment (start 72.39 71.258488) (end 75.264641 74.133129) (width 0.254) (layer F.Cu) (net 35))
 (segment (start 72.39 66.04) (end 72.39 71.258488) (width 0.254) (layer F.Cu) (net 35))
 (segment (start 68.58 64.77) (end 71.755 67.945) (width 0.254) (layer F.Cu) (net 36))
 (segment (start 71.755 71.755) (end 74.698885 74.698885) (width 0.254) (layer F.Cu) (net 36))
 (segment (start 71.755 67.945) (end 71.755 71.755) (width 0.254) (layer F.Cu) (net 36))
 (segment (start 68.58 67.31) (end 71.12 69.85) (width 0.254) (layer F.Cu) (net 37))
 (segment (start 71.12 72.251512) (end 74.133129 75.264641) (width 0.254) (layer F.Cu) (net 37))
 (segment (start 71.12 69.85) (end 71.12 72.251512) (width 0.254) (layer F.Cu) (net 37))
 (segment (start 68.58 69.85) (end 70.485 71.755) (width 0.254) (layer F.Cu) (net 38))
 (segment (start 70.485 72.748025) (end 73.567372 75.830397) (width 0.254) (layer F.Cu) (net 38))
 (segment (start 70.485 71.755) (end 70.485 72.748025) (width 0.254) (layer F.Cu) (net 38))
 (segment (start 88.9 74.93) (end 87.076049 74.93) (width 0.254) (layer F.Cu) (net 21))
 (segment (start 87.076049 74.93) (end 85.04414 76.961909) (width 0.254) (layer F.Cu) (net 21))
 (segment (start 88.9 52.07) (end 82.55 58.42) (width 0.254) (layer F.Cu) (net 30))
 (segment (start 82.55 69.272439) (end 79.952335 71.870104) (width 0.254) (layer F.Cu) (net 30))
 (segment (start 82.55 58.42) (end 82.55 69.272439) (width 0.254) (layer F.Cu) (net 30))
 (segment (start 83.185 69.768951) (end 80.518091 72.43586) (width 0.254) (layer F.Cu) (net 29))
 (segment (start 88.9 54.61) (end 83.185 60.325) (width 0.254) (layer F.Cu) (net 29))
 (segment (start 83.185 60.325) (end 83.185 69.768951) (width 0.254) (layer F.Cu) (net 29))
 (segment (start 86.36 72.251512) (end 83.346871 75.264641) (width 0.254) (layer F.Cu) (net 24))
 (segment (start 86.36 69.85) (end 86.36 72.251512) (width 0.254) (layer F.Cu) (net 24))
 (segment (start 88.9 67.31) (end 86.36 69.85) (width 0.254) (layer F.Cu) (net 24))
 (segment (start 86.995 72.748025) (end 83.912628 75.830397) (width 0.254) (layer F.Cu) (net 23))
 (segment (start 86.995 71.755) (end 86.995 72.748025) (width 0.254) (layer F.Cu) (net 23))
 (segment (start 88.9 69.85) (end 86.995 71.755) (width 0.254) (layer F.Cu) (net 23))
 (segment (start 73.344407 78.421159) (end 73.344407 78.478032) (width 0.254) (layer F.Cu) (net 9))
 (segment (start 73.344407 78.478032) (end 71.870104 79.952335) (width 0.254) (layer F.Cu) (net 9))
 (segment (start 71.870104 79.952335) (end 68.637665 79.952335) (width 0.254) (layer F.Cu) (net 9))
 (segment (start 68.637665 79.952335) (end 68.58 80.01) (width 0.254) (layer F.Cu) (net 9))
 (segment (start 88.484537 72.39) (end 84.478384 76.396153) (width 0.254) (layer F.Cu) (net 22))
 (segment (start 88.9 72.39) (end 88.484537 72.39) (width 0.254) (layer F.Cu) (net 22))
 (segment (start 88.9 105.41) (end 82.55 99.06) (width 0.254) (layer F.Cu) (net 17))
 (segment (start 82.55 88.207561) (end 79.952335 85.609896) (width 0.254) (layer F.Cu) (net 17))
 (segment (start 82.55 99.06) (end 82.55 88.207561) (width 0.254) (layer F.Cu) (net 17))
 (segment (start 68.58 52.07) (end 74.93 58.42) (width 0.254) (layer F.Cu) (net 31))
 (segment (start 74.93 69.272439) (end 77.527665 71.870104) (width 0.254) (layer F.Cu) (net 31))
 (segment (start 74.93 58.42) (end 74.93 69.272439) (width 0.254) (layer F.Cu) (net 31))
 (segment (start 68.58 54.61) (end 74.295 60.325) (width 0.254) (layer F.Cu) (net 32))
 (segment (start 74.295 69.768951) (end 76.961909 72.43586) (width 0.254) (layer F.Cu) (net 32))
 (segment (start 74.295 60.325) (end 74.295 69.768951) (width 0.254) (layer F.Cu) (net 32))
 (segment (start 68.58 57.15) (end 73.66 62.23) (width 0.254) (layer F.Cu) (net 33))
 (segment (start 73.66 70.265463) (end 76.396153 73.001616) (width 0.254) (layer F.Cu) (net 33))
 (segment (start 73.66 62.23) (end 73.66 70.265463) (width 0.254) (layer F.Cu) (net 33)))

